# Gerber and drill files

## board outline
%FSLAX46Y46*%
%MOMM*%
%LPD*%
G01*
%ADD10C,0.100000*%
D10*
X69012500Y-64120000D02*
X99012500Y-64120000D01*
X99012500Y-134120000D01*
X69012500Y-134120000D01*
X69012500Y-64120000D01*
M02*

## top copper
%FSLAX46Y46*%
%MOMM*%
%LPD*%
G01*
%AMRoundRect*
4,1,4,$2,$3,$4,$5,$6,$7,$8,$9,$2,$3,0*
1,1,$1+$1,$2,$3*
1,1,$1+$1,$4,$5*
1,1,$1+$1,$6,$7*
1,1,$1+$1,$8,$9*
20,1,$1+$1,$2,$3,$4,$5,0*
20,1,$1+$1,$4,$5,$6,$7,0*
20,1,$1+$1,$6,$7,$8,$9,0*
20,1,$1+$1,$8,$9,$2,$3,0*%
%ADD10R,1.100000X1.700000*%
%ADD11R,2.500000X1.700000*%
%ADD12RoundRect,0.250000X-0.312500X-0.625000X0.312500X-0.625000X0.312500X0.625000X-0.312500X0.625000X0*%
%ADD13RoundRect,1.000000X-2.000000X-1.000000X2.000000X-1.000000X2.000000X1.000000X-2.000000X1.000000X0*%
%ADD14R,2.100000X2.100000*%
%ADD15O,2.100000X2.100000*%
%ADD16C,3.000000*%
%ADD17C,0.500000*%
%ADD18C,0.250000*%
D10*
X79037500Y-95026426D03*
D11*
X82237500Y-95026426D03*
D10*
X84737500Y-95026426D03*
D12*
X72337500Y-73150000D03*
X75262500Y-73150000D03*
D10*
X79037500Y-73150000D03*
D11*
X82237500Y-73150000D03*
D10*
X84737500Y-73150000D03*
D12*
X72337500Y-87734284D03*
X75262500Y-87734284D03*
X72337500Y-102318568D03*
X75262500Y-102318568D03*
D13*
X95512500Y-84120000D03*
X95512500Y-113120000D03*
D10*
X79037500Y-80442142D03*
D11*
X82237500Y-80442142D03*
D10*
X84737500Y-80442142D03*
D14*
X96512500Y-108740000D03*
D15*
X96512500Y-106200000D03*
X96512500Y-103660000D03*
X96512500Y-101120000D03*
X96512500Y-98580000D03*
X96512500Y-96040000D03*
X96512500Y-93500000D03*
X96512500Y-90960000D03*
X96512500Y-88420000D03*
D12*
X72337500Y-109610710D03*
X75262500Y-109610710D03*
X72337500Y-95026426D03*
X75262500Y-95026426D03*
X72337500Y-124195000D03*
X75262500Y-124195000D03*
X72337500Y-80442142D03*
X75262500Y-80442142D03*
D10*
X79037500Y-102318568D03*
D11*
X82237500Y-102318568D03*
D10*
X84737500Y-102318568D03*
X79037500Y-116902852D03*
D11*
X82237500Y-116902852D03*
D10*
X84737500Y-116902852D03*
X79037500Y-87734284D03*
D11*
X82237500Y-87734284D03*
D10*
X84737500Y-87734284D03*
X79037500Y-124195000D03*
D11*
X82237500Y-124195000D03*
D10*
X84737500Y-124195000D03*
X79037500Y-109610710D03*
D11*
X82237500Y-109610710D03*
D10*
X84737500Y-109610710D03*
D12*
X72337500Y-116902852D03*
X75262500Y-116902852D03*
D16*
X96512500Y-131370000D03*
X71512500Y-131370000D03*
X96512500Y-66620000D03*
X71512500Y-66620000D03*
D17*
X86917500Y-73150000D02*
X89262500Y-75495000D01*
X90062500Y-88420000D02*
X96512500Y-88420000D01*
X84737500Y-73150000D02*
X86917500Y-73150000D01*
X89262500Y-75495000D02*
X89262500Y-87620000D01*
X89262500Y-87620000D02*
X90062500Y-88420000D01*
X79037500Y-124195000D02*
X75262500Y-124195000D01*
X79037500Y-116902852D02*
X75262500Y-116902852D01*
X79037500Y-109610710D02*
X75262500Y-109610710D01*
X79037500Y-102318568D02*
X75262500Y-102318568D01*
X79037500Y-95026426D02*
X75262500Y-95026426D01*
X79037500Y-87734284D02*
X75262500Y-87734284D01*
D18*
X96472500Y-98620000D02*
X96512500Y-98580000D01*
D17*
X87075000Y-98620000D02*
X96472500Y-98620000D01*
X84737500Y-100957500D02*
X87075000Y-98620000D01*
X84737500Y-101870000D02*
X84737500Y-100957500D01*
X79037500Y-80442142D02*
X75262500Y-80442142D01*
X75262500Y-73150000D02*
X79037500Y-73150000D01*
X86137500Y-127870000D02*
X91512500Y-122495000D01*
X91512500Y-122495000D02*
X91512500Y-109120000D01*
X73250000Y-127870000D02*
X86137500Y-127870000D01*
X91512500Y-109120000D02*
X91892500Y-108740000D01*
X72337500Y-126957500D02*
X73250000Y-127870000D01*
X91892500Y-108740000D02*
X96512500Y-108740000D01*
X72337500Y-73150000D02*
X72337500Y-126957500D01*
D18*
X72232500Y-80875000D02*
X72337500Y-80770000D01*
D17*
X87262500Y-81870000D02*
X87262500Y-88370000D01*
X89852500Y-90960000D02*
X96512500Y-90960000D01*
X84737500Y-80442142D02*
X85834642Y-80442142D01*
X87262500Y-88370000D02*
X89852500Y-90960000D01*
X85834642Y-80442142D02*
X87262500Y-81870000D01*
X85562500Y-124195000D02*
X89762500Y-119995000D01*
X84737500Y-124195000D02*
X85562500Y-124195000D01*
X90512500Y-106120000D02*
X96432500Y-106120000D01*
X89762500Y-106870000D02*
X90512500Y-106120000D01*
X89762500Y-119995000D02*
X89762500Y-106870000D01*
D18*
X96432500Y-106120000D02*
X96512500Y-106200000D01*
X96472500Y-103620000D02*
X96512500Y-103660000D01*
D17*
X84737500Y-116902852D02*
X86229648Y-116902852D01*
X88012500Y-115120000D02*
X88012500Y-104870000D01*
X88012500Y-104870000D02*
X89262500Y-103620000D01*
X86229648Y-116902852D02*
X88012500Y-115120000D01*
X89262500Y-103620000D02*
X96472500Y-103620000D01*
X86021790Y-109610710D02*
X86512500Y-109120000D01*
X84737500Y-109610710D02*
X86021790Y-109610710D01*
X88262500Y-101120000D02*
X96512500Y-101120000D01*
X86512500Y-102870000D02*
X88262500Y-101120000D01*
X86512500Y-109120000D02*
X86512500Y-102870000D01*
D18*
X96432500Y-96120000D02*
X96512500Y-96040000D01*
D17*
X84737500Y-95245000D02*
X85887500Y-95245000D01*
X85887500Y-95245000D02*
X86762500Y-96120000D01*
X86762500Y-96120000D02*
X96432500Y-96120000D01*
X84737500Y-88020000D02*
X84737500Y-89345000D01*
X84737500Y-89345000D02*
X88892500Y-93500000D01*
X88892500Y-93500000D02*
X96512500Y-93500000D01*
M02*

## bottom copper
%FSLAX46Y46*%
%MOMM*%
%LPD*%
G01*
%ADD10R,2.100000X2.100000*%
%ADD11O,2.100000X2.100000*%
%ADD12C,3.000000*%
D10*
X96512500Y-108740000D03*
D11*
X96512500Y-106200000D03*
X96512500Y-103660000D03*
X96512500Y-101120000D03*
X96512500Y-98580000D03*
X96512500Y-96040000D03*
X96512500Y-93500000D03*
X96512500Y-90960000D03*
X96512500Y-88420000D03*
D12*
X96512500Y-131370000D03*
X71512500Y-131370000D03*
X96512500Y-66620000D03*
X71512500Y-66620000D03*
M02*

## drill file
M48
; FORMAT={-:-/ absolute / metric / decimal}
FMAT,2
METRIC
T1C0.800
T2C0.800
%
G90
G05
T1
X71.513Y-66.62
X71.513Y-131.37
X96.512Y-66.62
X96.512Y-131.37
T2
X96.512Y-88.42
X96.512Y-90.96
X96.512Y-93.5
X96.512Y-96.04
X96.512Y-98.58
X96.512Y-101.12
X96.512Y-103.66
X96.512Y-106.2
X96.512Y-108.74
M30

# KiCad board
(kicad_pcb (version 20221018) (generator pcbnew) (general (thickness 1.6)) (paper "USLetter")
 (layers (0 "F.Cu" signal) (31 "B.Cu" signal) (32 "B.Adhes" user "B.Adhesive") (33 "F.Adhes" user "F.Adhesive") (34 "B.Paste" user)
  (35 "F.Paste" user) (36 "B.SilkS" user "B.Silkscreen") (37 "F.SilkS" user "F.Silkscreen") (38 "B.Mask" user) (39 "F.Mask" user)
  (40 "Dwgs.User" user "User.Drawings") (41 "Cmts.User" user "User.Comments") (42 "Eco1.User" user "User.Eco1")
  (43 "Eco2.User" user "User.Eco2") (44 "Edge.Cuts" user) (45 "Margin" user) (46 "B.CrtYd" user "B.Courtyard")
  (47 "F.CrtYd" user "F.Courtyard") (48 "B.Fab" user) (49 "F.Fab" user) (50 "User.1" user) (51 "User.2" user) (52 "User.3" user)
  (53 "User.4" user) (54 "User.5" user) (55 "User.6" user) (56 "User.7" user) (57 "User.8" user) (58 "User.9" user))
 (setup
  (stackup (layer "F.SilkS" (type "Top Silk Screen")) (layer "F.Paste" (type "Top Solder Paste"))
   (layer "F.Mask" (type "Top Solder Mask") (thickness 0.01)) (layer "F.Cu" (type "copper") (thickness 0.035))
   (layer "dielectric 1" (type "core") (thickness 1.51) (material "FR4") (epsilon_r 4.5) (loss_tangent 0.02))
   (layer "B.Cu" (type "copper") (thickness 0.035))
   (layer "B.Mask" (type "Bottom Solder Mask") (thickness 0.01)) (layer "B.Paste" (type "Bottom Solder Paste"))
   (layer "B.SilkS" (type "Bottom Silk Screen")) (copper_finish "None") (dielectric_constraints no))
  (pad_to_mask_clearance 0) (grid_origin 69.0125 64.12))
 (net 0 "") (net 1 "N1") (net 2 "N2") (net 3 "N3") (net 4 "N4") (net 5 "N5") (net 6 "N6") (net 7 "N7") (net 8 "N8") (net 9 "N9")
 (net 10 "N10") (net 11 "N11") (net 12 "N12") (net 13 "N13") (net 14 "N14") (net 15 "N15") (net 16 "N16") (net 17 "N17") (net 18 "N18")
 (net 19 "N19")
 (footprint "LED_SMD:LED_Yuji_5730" (layer "F.Cu") (at 81.8875 95.026426)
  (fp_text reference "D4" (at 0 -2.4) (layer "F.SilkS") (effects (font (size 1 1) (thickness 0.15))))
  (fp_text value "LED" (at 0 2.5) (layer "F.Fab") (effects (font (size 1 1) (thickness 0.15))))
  (pad "1" smd rect (at -2.85 0) (size 1.1 1.7) (layers "F.Cu" "F.Paste" "F.Mask") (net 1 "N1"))
  (pad "2" smd rect (at 0.35 0) (size 2.5 1.7) (layers "F.Cu" "F.Paste" "F.Mask") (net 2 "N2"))
  (pad "2" smd rect (at 2.85 0) (size 1.1 1.7) (layers "F.Cu" "F.Paste" "F.Mask") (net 2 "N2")))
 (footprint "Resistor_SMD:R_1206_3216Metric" (layer "F.Cu") (at 73.8 73.15)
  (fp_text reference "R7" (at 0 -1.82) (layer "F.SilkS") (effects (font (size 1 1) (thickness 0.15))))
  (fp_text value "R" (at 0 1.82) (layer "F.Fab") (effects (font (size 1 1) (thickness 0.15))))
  (pad "1" smd roundrect (at -1.4625 0) (size 1.125 1.75) (layers "F.Cu" "F.Paste" "F.Mask") (roundrect_rratio 0.2222222222) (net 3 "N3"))
  (pad "2" smd roundrect (at 1.4625 0) (size 1.125 1.75) (layers "F.Cu" "F.Paste" "F.Mask") (roundrect_rratio 0.2222222222) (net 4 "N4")))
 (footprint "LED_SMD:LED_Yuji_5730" (layer "F.Cu") (at 81.8875 73.15)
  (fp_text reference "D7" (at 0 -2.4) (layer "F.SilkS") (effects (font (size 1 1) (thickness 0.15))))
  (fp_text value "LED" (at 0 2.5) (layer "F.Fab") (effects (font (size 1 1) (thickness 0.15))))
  (pad "1" smd rect (at -2.85 0) (size 1.1 1.7) (layers "F.Cu" "F.Paste" "F.Mask") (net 4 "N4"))
  (pad "2" smd rect (at 0.35 0) (size 2.5 1.7) (layers "F.Cu" "F.Paste" "F.Mask") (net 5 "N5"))
  (pad "2" smd rect (at 2.85 0) (size 1.1 1.7) (layers "F.Cu" "F.Paste" "F.Mask") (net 5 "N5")))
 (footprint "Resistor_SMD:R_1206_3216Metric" (layer "F.Cu") (at 73.8 87.734284)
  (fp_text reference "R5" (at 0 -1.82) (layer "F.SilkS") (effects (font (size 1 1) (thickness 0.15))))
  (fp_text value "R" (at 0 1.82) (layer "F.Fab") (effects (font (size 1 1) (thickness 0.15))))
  (pad "1" smd roundrect (at -1.4625 0) (size 1.125 1.75) (layers "F.Cu" "F.Paste" "F.Mask") (roundrect_rratio 0.2222222222) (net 3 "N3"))
  (pad "2" smd roundrect (at 1.4625 0) (size 1.125 1.75) (layers "F.Cu" "F.Paste" "F.Mask") (roundrect_rratio 0.2222222222) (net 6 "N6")))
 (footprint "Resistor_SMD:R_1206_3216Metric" (layer "F.Cu") (at 73.8 102.318568)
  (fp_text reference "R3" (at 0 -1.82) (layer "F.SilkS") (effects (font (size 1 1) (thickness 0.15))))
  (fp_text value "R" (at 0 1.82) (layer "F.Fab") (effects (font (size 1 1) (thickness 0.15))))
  (pad "1" smd roundrect (at -1.4625 0) (size 1.125 1.75) (layers "F.Cu" "F.Paste" "F.Mask") (roundrect_rratio 0.2222222222) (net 3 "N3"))
  (pad "2" smd roundrect (at 1.4625 0) (size 1.125 1.75) (layers "F.Cu" "F.Paste" "F.Mask") (roundrect_rratio 0.2222222222) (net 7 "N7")))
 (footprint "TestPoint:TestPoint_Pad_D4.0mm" (layer "F.Cu") (at 95.5125 84.12)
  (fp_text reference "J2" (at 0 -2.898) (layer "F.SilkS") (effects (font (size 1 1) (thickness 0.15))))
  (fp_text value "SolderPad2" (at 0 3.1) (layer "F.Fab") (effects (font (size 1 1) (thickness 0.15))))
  (pad "1" smd roundrect (at 0 0) (size 6 4) (layers "F.Cu" "F.Mask") (roundrect_rratio 0.25) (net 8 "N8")))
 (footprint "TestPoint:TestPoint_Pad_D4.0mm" (layer "F.Cu") (at 95.5125 113.12)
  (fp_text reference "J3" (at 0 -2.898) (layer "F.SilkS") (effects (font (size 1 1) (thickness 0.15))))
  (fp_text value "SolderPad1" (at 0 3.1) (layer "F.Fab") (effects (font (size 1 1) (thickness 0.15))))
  (pad "1" smd roundrect (at 0 0) (size 6 4) (layers "F.Cu" "F.Mask") (roundrect_rratio 0.25) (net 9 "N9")))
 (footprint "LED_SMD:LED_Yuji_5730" (layer "F.Cu") (at 81.8875 80.442142)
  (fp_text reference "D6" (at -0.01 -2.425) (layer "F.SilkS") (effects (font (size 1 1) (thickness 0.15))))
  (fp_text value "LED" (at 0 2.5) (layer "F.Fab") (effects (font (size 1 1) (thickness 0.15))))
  (pad "1" smd rect (at -2.85 0) (size 1.1 1.7) (layers "F.Cu" "F.Paste" "F.Mask") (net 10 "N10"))
  (pad "2" smd rect (at 0.35 0) (size 2.5 1.7) (layers "F.Cu" "F.Paste" "F.Mask") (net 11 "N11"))
  (pad "2" smd rect (at 2.85 0) (size 1.1 1.7) (layers "F.Cu" "F.Paste" "F.Mask") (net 11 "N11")))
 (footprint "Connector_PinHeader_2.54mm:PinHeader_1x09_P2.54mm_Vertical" (layer "F.Cu") (at 96.5125 108.74 180)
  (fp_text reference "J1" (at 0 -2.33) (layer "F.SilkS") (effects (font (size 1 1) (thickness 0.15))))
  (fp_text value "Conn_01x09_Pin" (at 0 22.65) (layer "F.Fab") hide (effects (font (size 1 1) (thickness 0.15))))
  (pad "1" thru_hole rect (at 0 0 180) (size 2.1 2.1) (drill 0.8) (layers "*.Cu" "*.Mask") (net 3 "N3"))
  (pad "2" thru_hole oval (at 0 2.54 180) (size 2.1 2.1) (drill 0.8) (layers "*.Cu" "*.Mask") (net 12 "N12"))
  (pad "3" thru_hole oval (at 0 5.08 180) (size 2.1 2.1) (drill 0.8) (layers "*.Cu" "*.Mask") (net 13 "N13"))
  (pad "4" thru_hole oval (at 0 7.62 180) (size 2.1 2.1) (drill 0.8) (layers "*.Cu" "*.Mask") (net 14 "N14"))
  (pad "5" thru_hole oval (at 0 10.16 180) (size 2.1 2.1) (drill 0.8) (layers "*.Cu" "*.Mask") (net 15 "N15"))
  (pad "6" thru_hole oval (at 0 12.7 180) (size 2.1 2.1) (drill 0.8) (layers "*.Cu" "*.Mask") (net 2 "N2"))
  (pad "7" thru_hole oval (at 0 15.24 180) (size 2.1 2.1) (drill 0.8) (layers "*.Cu" "*.Mask") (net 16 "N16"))
  (pad "8" thru_hole oval (at 0 17.78 180) (size 2.1 2.1) (drill 0.8) (layers "*.Cu" "*.Mask") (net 11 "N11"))
  (pad "9" thru_hole oval (at 0 20.32 180) (size 2.1 2.1) (drill 0.8) (layers "*.Cu" "*.Mask") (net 5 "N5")))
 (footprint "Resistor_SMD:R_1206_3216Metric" (layer "F.Cu") (at 73.8 109.61071)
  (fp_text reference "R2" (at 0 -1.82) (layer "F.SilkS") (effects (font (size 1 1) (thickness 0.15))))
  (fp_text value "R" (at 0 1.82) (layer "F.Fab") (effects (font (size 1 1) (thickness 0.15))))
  (pad "1" smd roundrect (at -1.4625 0) (size 1.125 1.75) (layers "F.Cu" "F.Paste" "F.Mask") (roundrect_rratio 0.2222222222) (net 3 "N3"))
  (pad "2" smd roundrect (at 1.4625 0) (size 1.125 1.75) (layers "F.Cu" "F.Paste" "F.Mask") (roundrect_rratio 0.2222222222) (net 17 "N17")))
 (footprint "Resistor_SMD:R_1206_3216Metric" (layer "F.Cu") (at 73.8 95.026426)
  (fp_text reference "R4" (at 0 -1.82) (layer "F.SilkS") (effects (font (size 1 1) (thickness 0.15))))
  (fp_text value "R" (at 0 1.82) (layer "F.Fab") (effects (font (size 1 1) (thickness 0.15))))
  (pad "1" smd roundrect (at -1.4625 0) (size 1.125 1.75) (layers "F.Cu" "F.Paste" "F.Mask") (roundrect_rratio 0.2222222222) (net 3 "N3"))
  (pad "2" smd roundrect (at 1.4625 0) (size 1.125 1.75) (layers "F.Cu" "F.Paste" "F.Mask") (roundrect_rratio 0.2222222222) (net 1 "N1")))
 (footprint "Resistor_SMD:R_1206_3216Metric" (layer "F.Cu") (at 73.8 124.195)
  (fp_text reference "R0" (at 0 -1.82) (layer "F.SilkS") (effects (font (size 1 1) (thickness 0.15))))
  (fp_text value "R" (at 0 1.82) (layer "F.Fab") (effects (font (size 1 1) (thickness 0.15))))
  (pad "1" smd roundrect (at -1.4625 0) (size 1.125 1.75) (layers "F.Cu" "F.Paste" "F.Mask") (roundrect_rratio 0.2222222222) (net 3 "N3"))
  (pad "2" smd roundrect (at 1.4625 0) (size 1.125 1.75) (layers "F.Cu" "F.Paste" "F.Mask") (roundrect_rratio 0.2222222222) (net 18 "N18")))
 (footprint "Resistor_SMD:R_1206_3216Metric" (layer "F.Cu") (at 73.8 80.442142)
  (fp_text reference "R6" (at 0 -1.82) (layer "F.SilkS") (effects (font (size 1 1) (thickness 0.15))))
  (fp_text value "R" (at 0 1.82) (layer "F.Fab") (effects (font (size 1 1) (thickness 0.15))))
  (pad "1" smd roundrect (at -1.4625 0) (size 1.125 1.75) (layers "F.Cu" "F.Paste" "F.Mask") (roundrect_rratio 0.2222222222) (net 3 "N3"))
  (pad "2" smd roundrect (at 1.4625 0) (size 1.125 1.75) (layers "F.Cu" "F.Paste" "F.Mask") (roundrect_rratio 0.2222222222) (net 10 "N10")))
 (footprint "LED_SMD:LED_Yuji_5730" (layer "F.Cu") (at 81.8875 102.318568)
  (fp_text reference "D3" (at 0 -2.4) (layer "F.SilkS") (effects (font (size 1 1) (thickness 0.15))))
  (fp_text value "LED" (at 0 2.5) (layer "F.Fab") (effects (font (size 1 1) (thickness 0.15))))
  (pad "1" smd rect (at -2.85 0) (size 1.1 1.7) (layers "F.Cu" "F.Paste" "F.Mask") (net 7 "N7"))
  (pad "2" smd rect (at 0.35 0) (size 2.5 1.7) (layers "F.Cu" "F.Paste" "F.Mask") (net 15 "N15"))
  (pad "2" smd rect (at 2.85 0) (size 1.1 1.7) (layers "F.Cu" "F.Paste" "F.Mask") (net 15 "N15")))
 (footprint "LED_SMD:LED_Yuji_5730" (layer "F.Cu") (at 81.8875 116.902852)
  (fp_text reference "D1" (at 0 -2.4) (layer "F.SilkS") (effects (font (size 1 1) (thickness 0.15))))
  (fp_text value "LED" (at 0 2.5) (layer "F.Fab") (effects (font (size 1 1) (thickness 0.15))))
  (pad "1" smd rect (at -2.85 0) (size 1.1 1.7) (layers "F.Cu" "F.Paste" "F.Mask") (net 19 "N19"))
  (pad "2" smd rect (at 0.35 0) (size 2.5 1.7) (layers "F.Cu" "F.Paste" "F.Mask") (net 13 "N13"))
  (pad "2" smd rect (at 2.85 0) (size 1.1 1.7) (layers "F.Cu" "F.Paste" "F.Mask") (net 13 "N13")))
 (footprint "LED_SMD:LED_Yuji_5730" (layer "F.Cu") (at 81.8875 87.734284)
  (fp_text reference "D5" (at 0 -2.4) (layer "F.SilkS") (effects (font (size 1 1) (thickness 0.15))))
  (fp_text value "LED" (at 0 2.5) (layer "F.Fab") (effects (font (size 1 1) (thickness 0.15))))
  (pad "1" smd rect (at -2.85 0) (size 1.1 1.7) (layers "F.Cu" "F.Paste" "F.Mask") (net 6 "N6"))
  (pad "2" smd rect (at 0.35 0) (size 2.5 1.7) (layers "F.Cu" "F.Paste" "F.Mask") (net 16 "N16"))
  (pad "2" smd rect (at 2.85 0) (size 1.1 1.7) (layers "F.Cu" "F.Paste" "F.Mask") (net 16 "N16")))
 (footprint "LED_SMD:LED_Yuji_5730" (layer "F.Cu") (at 81.8875 124.195)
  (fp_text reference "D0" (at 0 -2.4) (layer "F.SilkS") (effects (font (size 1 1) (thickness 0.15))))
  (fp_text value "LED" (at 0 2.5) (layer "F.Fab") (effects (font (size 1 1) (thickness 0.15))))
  (pad "1" smd rect (at -2.85 0) (size 1.1 1.7) (layers "F.Cu" "F.Paste" "F.Mask") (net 18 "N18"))
  (pad "2" smd rect (at 0.35 0) (size 2.5 1.7) (layers "F.Cu" "F.Paste" "F.Mask") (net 12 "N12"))
  (pad "2" smd rect (at 2.85 0) (size 1.1 1.7) (layers "F.Cu" "F.Paste" "F.Mask") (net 12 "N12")))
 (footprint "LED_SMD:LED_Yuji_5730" (layer "F.Cu") (at 81.8875 109.61071)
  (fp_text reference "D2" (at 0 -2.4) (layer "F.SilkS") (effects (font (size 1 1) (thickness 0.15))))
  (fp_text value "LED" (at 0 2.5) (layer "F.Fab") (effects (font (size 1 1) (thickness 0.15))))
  (pad "1" smd rect (at -2.85 0) (size 1.1 1.7) (layers "F.Cu" "F.Paste" "F.Mask") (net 17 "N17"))
  (pad "2" smd rect (at 0.35 0) (size 2.5 1.7) (layers "F.Cu" "F.Paste" "F.Mask") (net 14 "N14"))
  (pad "2" smd rect (at 2.85 0) (size 1.1 1.7) (layers "F.Cu" "F.Paste" "F.Mask") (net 14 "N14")))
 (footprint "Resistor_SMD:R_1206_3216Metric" (layer "F.Cu") (at 73.8 116.902852)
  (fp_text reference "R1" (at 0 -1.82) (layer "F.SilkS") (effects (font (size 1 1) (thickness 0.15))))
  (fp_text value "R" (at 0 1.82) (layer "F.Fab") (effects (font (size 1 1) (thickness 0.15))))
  (pad "1" smd roundrect (at -1.4625 0) (size 1.125 1.75) (layers "F.Cu" "F.Paste" "F.Mask") (roundrect_rratio 0.2222222222) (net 3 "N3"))
  (pad "2" smd roundrect (at 1.4625 0) (size 1.125 1.75) (layers "F.Cu" "F.Paste" "F.Mask") (roundrect_rratio 0.2222222222) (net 19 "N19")))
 (gr_rect (start 69.0125 64.12) (end 99.0125 134.12) (stroke (width 0.1) (type default)) (fill none) (layer "Edge.Cuts"))
 (via (at 96.5125 131.37) (size 3) (drill 0.8) (layers "F.Cu" "B.Cu") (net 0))
 (via (at 71.5125 131.37) (size 3) (drill 0.8) (layers "F.Cu" "B.Cu") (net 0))
 (via (at 96.5125 66.62) (size 3) (drill 0.8) (layers "F.Cu" "B.Cu") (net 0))
 (via (at 71.5125 66.62) (size 3) (drill 0.8) (layers "F.Cu" "B.Cu") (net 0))
 (segment (start 86.9175 73.15) (end 89.2625 75.495) (width 0.5) (layer "F.Cu") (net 5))
 (segment (start 90.0625 88.42) (end 96.5125 88.42) (width 0.5) (layer "F.Cu") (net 5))
 (segment (start 84.7375 73.15) (end 86.9175 73.15) (width 0.5) (layer "F.Cu") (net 5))
 (segment (start 89.2625 75.495) (end 89.2625 87.62) (width 0.5) (layer "F.Cu") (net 5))
 (segment (start 89.2625 87.62) (end 90.0625 88.42) (width 0.5) (layer "F.Cu") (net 5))
 (segment (start 79.0375 124.195) (end 75.2625 124.195) (width 0.5) (layer "F.Cu") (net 18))
 (segment (start 79.0375 116.902852) (end 75.2625 116.902852) (width 0.5) (layer "F.Cu") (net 19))
 (segment (start 79.0375 109.61071) (end 75.2625 109.61071) (width 0.5) (layer "F.Cu") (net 17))
 (segment (start 79.0375 102.318568) (end 75.2625 102.318568) (width 0.5) (layer "F.Cu") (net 7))
 (segment (start 79.0375 95.026426) (end 75.2625 95.026426) (width 0.5) (layer "F.Cu") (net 1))
 (segment (start 79.0375 87.734284) (end 75.2625 87.734284) (width 0.5) (layer "F.Cu") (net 6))
 (segment (start 96.4725 98.62) (end 96.5125 98.58) (width 0.25) (layer "F.Cu") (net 15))
 (segment (start 87.075 98.62) (end 96.4725 98.62) (width 0.5) (layer "F.Cu") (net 15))
 (segment (start 84.7375 100.9575) (end 87.075 98.62) (width 0.5) (layer "F.Cu") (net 15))
 (segment (start 84.7375 101.87) (end 84.7375 100.9575) (width 0.5) (layer "F.Cu") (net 15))
 (segment (start 79.0375 80.442142) (end 75.2625 80.442142) (width 0.5) (layer "F.Cu") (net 10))
 (segment (start 75.2625 73.15) (end 79.0375 73.15) (width 0.5) (layer "F.Cu") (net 4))
 (segment (start 86.1375 127.87) (end 91.5125 122.495) (width 0.5) (layer "F.Cu") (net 3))
 (segment (start 91.5125 122.495) (end 91.5125 109.12) (width 0.5) (layer "F.Cu") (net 3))
 (segment (start 73.25 127.87) (end 86.1375 127.87) (width 0.5) (layer "F.Cu") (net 3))
 (segment (start 91.5125 109.12) (end 91.8925 108.74) (width 0.5) (layer "F.Cu") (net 3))
 (segment (start 72.3375 126.9575) (end 73.25 127.87) (width 0.5) (layer "F.Cu") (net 3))
 (segment (start 91.8925 108.74) (end 96.5125 108.74) (width 0.5) (layer "F.Cu") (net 3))
 (segment (start 72.3375 73.15) (end 72.3375 126.9575) (width 0.5) (layer "F.Cu") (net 3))
 (segment (start 72.2325 80.875) (end 72.3375 80.77) (width 0.25) (layer "F.Cu") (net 3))
 (segment (start 87.2625 81.87) (end 87.2625 88.37) (width 0.5) (layer "F.Cu") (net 11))
 (segment (start 89.8525 90.96) (end 96.5125 90.96) (width 0.5) (layer "F.Cu") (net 11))
 (segment (start 84.7375 80.442142) (end 85.834642 80.442142) (width 0.5) (layer "F.Cu") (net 11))
 (segment (start 87.2625 88.37) (end 89.8525 90.96) (width 0.5) (layer "F.Cu") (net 11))
 (segment (start 85.834642 80.442142) (end 87.2625 81.87) (width 0.5) (layer "F.Cu") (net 11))
 (segment (start 85.5625 124.195) (end 89.7625 119.995) (width 0.5) (layer "F.Cu") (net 12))
 (segment (start 84.7375 124.195) (end 85.5625 124.195) (width 0.5) (layer "F.Cu") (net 12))
 (segment (start 90.5125 106.12) (end 96.4325 106.12) (width 0.5) (layer "F.Cu") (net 12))
 (segment (start 89.7625 106.87) (end 90.5125 106.12) (width 0.5) (layer "F.Cu") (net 12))
 (segment (start 89.7625 119.995) (end 89.7625 106.87) (width 0.5) (layer "F.Cu") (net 12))
 (segment (start 96.4325 106.12) (end 96.5125 106.2) (width 0.25) (layer "F.Cu") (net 12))
 (segment (start 96.4725 103.62) (end 96.5125 103.66) (width 0.25) (layer "F.Cu") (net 13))
 (segment (start 84.7375 116.902852) (end 86.229648 116.902852) (width 0.5) (layer "F.Cu") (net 13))
 (segment (start 88.0125 115.12) (end 88.0125 104.87) (width 0.5) (layer "F.Cu") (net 13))
 (segment (start 88.0125 104.87) (end 89.2625 103.62) (width 0.5) (layer "F.Cu") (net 13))
 (segment (start 86.229648 116.902852) (end 88.0125 115.12) (width 0.5) (layer "F.Cu") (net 13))
 (segment (start 89.2625 103.62) (end 96.4725 103.62) (width 0.5) (layer "F.Cu") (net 13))
 (segment (start 86.02179 109.61071) (end 86.5125 109.12) (width 0.5) (layer "F.Cu") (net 14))
 (segment (start 84.7375 109.61071) (end 86.02179 109.61071) (width 0.5) (layer "F.Cu") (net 14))
 (segment (start 88.2625 101.12) (end 96.5125 101.12) (width 0.5) (layer "F.Cu") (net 14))
 (segment (start 86.5125 102.87) (end 88.2625 101.12) (width 0.5) (layer "F.Cu") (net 14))
 (segment (start 86.5125 109.12) (end 86.5125 102.87) (width 0.5) (layer "F.Cu") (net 14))
 (segment (start 96.4325 96.12) (end 96.5125 96.04) (width 0.25) (layer "F.Cu") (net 2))
 (segment (start 84.7375 95.245) (end 85.8875 95.245) (width 0.5) (layer "F.Cu") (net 2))
 (segment (start 85.8875 95.245) (end 86.7625 96.12) (width 0.5) (layer "F.Cu") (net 2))
 (segment (start 86.7625 96.12) (end 96.4325 96.12) (width 0.5) (layer "F.Cu") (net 2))
 (segment (start 84.7375 88.02) (end 84.7375 89.345) (width 0.5) (layer "F.Cu") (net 16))
 (segment (start 84.7375 89.345) (end 88.8925 93.5) (width 0.5) (layer "F.Cu") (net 16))
 (segment (start 88.8925 93.5) (end 96.5125 93.5) (width 0.5) (layer "F.Cu") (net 16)))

